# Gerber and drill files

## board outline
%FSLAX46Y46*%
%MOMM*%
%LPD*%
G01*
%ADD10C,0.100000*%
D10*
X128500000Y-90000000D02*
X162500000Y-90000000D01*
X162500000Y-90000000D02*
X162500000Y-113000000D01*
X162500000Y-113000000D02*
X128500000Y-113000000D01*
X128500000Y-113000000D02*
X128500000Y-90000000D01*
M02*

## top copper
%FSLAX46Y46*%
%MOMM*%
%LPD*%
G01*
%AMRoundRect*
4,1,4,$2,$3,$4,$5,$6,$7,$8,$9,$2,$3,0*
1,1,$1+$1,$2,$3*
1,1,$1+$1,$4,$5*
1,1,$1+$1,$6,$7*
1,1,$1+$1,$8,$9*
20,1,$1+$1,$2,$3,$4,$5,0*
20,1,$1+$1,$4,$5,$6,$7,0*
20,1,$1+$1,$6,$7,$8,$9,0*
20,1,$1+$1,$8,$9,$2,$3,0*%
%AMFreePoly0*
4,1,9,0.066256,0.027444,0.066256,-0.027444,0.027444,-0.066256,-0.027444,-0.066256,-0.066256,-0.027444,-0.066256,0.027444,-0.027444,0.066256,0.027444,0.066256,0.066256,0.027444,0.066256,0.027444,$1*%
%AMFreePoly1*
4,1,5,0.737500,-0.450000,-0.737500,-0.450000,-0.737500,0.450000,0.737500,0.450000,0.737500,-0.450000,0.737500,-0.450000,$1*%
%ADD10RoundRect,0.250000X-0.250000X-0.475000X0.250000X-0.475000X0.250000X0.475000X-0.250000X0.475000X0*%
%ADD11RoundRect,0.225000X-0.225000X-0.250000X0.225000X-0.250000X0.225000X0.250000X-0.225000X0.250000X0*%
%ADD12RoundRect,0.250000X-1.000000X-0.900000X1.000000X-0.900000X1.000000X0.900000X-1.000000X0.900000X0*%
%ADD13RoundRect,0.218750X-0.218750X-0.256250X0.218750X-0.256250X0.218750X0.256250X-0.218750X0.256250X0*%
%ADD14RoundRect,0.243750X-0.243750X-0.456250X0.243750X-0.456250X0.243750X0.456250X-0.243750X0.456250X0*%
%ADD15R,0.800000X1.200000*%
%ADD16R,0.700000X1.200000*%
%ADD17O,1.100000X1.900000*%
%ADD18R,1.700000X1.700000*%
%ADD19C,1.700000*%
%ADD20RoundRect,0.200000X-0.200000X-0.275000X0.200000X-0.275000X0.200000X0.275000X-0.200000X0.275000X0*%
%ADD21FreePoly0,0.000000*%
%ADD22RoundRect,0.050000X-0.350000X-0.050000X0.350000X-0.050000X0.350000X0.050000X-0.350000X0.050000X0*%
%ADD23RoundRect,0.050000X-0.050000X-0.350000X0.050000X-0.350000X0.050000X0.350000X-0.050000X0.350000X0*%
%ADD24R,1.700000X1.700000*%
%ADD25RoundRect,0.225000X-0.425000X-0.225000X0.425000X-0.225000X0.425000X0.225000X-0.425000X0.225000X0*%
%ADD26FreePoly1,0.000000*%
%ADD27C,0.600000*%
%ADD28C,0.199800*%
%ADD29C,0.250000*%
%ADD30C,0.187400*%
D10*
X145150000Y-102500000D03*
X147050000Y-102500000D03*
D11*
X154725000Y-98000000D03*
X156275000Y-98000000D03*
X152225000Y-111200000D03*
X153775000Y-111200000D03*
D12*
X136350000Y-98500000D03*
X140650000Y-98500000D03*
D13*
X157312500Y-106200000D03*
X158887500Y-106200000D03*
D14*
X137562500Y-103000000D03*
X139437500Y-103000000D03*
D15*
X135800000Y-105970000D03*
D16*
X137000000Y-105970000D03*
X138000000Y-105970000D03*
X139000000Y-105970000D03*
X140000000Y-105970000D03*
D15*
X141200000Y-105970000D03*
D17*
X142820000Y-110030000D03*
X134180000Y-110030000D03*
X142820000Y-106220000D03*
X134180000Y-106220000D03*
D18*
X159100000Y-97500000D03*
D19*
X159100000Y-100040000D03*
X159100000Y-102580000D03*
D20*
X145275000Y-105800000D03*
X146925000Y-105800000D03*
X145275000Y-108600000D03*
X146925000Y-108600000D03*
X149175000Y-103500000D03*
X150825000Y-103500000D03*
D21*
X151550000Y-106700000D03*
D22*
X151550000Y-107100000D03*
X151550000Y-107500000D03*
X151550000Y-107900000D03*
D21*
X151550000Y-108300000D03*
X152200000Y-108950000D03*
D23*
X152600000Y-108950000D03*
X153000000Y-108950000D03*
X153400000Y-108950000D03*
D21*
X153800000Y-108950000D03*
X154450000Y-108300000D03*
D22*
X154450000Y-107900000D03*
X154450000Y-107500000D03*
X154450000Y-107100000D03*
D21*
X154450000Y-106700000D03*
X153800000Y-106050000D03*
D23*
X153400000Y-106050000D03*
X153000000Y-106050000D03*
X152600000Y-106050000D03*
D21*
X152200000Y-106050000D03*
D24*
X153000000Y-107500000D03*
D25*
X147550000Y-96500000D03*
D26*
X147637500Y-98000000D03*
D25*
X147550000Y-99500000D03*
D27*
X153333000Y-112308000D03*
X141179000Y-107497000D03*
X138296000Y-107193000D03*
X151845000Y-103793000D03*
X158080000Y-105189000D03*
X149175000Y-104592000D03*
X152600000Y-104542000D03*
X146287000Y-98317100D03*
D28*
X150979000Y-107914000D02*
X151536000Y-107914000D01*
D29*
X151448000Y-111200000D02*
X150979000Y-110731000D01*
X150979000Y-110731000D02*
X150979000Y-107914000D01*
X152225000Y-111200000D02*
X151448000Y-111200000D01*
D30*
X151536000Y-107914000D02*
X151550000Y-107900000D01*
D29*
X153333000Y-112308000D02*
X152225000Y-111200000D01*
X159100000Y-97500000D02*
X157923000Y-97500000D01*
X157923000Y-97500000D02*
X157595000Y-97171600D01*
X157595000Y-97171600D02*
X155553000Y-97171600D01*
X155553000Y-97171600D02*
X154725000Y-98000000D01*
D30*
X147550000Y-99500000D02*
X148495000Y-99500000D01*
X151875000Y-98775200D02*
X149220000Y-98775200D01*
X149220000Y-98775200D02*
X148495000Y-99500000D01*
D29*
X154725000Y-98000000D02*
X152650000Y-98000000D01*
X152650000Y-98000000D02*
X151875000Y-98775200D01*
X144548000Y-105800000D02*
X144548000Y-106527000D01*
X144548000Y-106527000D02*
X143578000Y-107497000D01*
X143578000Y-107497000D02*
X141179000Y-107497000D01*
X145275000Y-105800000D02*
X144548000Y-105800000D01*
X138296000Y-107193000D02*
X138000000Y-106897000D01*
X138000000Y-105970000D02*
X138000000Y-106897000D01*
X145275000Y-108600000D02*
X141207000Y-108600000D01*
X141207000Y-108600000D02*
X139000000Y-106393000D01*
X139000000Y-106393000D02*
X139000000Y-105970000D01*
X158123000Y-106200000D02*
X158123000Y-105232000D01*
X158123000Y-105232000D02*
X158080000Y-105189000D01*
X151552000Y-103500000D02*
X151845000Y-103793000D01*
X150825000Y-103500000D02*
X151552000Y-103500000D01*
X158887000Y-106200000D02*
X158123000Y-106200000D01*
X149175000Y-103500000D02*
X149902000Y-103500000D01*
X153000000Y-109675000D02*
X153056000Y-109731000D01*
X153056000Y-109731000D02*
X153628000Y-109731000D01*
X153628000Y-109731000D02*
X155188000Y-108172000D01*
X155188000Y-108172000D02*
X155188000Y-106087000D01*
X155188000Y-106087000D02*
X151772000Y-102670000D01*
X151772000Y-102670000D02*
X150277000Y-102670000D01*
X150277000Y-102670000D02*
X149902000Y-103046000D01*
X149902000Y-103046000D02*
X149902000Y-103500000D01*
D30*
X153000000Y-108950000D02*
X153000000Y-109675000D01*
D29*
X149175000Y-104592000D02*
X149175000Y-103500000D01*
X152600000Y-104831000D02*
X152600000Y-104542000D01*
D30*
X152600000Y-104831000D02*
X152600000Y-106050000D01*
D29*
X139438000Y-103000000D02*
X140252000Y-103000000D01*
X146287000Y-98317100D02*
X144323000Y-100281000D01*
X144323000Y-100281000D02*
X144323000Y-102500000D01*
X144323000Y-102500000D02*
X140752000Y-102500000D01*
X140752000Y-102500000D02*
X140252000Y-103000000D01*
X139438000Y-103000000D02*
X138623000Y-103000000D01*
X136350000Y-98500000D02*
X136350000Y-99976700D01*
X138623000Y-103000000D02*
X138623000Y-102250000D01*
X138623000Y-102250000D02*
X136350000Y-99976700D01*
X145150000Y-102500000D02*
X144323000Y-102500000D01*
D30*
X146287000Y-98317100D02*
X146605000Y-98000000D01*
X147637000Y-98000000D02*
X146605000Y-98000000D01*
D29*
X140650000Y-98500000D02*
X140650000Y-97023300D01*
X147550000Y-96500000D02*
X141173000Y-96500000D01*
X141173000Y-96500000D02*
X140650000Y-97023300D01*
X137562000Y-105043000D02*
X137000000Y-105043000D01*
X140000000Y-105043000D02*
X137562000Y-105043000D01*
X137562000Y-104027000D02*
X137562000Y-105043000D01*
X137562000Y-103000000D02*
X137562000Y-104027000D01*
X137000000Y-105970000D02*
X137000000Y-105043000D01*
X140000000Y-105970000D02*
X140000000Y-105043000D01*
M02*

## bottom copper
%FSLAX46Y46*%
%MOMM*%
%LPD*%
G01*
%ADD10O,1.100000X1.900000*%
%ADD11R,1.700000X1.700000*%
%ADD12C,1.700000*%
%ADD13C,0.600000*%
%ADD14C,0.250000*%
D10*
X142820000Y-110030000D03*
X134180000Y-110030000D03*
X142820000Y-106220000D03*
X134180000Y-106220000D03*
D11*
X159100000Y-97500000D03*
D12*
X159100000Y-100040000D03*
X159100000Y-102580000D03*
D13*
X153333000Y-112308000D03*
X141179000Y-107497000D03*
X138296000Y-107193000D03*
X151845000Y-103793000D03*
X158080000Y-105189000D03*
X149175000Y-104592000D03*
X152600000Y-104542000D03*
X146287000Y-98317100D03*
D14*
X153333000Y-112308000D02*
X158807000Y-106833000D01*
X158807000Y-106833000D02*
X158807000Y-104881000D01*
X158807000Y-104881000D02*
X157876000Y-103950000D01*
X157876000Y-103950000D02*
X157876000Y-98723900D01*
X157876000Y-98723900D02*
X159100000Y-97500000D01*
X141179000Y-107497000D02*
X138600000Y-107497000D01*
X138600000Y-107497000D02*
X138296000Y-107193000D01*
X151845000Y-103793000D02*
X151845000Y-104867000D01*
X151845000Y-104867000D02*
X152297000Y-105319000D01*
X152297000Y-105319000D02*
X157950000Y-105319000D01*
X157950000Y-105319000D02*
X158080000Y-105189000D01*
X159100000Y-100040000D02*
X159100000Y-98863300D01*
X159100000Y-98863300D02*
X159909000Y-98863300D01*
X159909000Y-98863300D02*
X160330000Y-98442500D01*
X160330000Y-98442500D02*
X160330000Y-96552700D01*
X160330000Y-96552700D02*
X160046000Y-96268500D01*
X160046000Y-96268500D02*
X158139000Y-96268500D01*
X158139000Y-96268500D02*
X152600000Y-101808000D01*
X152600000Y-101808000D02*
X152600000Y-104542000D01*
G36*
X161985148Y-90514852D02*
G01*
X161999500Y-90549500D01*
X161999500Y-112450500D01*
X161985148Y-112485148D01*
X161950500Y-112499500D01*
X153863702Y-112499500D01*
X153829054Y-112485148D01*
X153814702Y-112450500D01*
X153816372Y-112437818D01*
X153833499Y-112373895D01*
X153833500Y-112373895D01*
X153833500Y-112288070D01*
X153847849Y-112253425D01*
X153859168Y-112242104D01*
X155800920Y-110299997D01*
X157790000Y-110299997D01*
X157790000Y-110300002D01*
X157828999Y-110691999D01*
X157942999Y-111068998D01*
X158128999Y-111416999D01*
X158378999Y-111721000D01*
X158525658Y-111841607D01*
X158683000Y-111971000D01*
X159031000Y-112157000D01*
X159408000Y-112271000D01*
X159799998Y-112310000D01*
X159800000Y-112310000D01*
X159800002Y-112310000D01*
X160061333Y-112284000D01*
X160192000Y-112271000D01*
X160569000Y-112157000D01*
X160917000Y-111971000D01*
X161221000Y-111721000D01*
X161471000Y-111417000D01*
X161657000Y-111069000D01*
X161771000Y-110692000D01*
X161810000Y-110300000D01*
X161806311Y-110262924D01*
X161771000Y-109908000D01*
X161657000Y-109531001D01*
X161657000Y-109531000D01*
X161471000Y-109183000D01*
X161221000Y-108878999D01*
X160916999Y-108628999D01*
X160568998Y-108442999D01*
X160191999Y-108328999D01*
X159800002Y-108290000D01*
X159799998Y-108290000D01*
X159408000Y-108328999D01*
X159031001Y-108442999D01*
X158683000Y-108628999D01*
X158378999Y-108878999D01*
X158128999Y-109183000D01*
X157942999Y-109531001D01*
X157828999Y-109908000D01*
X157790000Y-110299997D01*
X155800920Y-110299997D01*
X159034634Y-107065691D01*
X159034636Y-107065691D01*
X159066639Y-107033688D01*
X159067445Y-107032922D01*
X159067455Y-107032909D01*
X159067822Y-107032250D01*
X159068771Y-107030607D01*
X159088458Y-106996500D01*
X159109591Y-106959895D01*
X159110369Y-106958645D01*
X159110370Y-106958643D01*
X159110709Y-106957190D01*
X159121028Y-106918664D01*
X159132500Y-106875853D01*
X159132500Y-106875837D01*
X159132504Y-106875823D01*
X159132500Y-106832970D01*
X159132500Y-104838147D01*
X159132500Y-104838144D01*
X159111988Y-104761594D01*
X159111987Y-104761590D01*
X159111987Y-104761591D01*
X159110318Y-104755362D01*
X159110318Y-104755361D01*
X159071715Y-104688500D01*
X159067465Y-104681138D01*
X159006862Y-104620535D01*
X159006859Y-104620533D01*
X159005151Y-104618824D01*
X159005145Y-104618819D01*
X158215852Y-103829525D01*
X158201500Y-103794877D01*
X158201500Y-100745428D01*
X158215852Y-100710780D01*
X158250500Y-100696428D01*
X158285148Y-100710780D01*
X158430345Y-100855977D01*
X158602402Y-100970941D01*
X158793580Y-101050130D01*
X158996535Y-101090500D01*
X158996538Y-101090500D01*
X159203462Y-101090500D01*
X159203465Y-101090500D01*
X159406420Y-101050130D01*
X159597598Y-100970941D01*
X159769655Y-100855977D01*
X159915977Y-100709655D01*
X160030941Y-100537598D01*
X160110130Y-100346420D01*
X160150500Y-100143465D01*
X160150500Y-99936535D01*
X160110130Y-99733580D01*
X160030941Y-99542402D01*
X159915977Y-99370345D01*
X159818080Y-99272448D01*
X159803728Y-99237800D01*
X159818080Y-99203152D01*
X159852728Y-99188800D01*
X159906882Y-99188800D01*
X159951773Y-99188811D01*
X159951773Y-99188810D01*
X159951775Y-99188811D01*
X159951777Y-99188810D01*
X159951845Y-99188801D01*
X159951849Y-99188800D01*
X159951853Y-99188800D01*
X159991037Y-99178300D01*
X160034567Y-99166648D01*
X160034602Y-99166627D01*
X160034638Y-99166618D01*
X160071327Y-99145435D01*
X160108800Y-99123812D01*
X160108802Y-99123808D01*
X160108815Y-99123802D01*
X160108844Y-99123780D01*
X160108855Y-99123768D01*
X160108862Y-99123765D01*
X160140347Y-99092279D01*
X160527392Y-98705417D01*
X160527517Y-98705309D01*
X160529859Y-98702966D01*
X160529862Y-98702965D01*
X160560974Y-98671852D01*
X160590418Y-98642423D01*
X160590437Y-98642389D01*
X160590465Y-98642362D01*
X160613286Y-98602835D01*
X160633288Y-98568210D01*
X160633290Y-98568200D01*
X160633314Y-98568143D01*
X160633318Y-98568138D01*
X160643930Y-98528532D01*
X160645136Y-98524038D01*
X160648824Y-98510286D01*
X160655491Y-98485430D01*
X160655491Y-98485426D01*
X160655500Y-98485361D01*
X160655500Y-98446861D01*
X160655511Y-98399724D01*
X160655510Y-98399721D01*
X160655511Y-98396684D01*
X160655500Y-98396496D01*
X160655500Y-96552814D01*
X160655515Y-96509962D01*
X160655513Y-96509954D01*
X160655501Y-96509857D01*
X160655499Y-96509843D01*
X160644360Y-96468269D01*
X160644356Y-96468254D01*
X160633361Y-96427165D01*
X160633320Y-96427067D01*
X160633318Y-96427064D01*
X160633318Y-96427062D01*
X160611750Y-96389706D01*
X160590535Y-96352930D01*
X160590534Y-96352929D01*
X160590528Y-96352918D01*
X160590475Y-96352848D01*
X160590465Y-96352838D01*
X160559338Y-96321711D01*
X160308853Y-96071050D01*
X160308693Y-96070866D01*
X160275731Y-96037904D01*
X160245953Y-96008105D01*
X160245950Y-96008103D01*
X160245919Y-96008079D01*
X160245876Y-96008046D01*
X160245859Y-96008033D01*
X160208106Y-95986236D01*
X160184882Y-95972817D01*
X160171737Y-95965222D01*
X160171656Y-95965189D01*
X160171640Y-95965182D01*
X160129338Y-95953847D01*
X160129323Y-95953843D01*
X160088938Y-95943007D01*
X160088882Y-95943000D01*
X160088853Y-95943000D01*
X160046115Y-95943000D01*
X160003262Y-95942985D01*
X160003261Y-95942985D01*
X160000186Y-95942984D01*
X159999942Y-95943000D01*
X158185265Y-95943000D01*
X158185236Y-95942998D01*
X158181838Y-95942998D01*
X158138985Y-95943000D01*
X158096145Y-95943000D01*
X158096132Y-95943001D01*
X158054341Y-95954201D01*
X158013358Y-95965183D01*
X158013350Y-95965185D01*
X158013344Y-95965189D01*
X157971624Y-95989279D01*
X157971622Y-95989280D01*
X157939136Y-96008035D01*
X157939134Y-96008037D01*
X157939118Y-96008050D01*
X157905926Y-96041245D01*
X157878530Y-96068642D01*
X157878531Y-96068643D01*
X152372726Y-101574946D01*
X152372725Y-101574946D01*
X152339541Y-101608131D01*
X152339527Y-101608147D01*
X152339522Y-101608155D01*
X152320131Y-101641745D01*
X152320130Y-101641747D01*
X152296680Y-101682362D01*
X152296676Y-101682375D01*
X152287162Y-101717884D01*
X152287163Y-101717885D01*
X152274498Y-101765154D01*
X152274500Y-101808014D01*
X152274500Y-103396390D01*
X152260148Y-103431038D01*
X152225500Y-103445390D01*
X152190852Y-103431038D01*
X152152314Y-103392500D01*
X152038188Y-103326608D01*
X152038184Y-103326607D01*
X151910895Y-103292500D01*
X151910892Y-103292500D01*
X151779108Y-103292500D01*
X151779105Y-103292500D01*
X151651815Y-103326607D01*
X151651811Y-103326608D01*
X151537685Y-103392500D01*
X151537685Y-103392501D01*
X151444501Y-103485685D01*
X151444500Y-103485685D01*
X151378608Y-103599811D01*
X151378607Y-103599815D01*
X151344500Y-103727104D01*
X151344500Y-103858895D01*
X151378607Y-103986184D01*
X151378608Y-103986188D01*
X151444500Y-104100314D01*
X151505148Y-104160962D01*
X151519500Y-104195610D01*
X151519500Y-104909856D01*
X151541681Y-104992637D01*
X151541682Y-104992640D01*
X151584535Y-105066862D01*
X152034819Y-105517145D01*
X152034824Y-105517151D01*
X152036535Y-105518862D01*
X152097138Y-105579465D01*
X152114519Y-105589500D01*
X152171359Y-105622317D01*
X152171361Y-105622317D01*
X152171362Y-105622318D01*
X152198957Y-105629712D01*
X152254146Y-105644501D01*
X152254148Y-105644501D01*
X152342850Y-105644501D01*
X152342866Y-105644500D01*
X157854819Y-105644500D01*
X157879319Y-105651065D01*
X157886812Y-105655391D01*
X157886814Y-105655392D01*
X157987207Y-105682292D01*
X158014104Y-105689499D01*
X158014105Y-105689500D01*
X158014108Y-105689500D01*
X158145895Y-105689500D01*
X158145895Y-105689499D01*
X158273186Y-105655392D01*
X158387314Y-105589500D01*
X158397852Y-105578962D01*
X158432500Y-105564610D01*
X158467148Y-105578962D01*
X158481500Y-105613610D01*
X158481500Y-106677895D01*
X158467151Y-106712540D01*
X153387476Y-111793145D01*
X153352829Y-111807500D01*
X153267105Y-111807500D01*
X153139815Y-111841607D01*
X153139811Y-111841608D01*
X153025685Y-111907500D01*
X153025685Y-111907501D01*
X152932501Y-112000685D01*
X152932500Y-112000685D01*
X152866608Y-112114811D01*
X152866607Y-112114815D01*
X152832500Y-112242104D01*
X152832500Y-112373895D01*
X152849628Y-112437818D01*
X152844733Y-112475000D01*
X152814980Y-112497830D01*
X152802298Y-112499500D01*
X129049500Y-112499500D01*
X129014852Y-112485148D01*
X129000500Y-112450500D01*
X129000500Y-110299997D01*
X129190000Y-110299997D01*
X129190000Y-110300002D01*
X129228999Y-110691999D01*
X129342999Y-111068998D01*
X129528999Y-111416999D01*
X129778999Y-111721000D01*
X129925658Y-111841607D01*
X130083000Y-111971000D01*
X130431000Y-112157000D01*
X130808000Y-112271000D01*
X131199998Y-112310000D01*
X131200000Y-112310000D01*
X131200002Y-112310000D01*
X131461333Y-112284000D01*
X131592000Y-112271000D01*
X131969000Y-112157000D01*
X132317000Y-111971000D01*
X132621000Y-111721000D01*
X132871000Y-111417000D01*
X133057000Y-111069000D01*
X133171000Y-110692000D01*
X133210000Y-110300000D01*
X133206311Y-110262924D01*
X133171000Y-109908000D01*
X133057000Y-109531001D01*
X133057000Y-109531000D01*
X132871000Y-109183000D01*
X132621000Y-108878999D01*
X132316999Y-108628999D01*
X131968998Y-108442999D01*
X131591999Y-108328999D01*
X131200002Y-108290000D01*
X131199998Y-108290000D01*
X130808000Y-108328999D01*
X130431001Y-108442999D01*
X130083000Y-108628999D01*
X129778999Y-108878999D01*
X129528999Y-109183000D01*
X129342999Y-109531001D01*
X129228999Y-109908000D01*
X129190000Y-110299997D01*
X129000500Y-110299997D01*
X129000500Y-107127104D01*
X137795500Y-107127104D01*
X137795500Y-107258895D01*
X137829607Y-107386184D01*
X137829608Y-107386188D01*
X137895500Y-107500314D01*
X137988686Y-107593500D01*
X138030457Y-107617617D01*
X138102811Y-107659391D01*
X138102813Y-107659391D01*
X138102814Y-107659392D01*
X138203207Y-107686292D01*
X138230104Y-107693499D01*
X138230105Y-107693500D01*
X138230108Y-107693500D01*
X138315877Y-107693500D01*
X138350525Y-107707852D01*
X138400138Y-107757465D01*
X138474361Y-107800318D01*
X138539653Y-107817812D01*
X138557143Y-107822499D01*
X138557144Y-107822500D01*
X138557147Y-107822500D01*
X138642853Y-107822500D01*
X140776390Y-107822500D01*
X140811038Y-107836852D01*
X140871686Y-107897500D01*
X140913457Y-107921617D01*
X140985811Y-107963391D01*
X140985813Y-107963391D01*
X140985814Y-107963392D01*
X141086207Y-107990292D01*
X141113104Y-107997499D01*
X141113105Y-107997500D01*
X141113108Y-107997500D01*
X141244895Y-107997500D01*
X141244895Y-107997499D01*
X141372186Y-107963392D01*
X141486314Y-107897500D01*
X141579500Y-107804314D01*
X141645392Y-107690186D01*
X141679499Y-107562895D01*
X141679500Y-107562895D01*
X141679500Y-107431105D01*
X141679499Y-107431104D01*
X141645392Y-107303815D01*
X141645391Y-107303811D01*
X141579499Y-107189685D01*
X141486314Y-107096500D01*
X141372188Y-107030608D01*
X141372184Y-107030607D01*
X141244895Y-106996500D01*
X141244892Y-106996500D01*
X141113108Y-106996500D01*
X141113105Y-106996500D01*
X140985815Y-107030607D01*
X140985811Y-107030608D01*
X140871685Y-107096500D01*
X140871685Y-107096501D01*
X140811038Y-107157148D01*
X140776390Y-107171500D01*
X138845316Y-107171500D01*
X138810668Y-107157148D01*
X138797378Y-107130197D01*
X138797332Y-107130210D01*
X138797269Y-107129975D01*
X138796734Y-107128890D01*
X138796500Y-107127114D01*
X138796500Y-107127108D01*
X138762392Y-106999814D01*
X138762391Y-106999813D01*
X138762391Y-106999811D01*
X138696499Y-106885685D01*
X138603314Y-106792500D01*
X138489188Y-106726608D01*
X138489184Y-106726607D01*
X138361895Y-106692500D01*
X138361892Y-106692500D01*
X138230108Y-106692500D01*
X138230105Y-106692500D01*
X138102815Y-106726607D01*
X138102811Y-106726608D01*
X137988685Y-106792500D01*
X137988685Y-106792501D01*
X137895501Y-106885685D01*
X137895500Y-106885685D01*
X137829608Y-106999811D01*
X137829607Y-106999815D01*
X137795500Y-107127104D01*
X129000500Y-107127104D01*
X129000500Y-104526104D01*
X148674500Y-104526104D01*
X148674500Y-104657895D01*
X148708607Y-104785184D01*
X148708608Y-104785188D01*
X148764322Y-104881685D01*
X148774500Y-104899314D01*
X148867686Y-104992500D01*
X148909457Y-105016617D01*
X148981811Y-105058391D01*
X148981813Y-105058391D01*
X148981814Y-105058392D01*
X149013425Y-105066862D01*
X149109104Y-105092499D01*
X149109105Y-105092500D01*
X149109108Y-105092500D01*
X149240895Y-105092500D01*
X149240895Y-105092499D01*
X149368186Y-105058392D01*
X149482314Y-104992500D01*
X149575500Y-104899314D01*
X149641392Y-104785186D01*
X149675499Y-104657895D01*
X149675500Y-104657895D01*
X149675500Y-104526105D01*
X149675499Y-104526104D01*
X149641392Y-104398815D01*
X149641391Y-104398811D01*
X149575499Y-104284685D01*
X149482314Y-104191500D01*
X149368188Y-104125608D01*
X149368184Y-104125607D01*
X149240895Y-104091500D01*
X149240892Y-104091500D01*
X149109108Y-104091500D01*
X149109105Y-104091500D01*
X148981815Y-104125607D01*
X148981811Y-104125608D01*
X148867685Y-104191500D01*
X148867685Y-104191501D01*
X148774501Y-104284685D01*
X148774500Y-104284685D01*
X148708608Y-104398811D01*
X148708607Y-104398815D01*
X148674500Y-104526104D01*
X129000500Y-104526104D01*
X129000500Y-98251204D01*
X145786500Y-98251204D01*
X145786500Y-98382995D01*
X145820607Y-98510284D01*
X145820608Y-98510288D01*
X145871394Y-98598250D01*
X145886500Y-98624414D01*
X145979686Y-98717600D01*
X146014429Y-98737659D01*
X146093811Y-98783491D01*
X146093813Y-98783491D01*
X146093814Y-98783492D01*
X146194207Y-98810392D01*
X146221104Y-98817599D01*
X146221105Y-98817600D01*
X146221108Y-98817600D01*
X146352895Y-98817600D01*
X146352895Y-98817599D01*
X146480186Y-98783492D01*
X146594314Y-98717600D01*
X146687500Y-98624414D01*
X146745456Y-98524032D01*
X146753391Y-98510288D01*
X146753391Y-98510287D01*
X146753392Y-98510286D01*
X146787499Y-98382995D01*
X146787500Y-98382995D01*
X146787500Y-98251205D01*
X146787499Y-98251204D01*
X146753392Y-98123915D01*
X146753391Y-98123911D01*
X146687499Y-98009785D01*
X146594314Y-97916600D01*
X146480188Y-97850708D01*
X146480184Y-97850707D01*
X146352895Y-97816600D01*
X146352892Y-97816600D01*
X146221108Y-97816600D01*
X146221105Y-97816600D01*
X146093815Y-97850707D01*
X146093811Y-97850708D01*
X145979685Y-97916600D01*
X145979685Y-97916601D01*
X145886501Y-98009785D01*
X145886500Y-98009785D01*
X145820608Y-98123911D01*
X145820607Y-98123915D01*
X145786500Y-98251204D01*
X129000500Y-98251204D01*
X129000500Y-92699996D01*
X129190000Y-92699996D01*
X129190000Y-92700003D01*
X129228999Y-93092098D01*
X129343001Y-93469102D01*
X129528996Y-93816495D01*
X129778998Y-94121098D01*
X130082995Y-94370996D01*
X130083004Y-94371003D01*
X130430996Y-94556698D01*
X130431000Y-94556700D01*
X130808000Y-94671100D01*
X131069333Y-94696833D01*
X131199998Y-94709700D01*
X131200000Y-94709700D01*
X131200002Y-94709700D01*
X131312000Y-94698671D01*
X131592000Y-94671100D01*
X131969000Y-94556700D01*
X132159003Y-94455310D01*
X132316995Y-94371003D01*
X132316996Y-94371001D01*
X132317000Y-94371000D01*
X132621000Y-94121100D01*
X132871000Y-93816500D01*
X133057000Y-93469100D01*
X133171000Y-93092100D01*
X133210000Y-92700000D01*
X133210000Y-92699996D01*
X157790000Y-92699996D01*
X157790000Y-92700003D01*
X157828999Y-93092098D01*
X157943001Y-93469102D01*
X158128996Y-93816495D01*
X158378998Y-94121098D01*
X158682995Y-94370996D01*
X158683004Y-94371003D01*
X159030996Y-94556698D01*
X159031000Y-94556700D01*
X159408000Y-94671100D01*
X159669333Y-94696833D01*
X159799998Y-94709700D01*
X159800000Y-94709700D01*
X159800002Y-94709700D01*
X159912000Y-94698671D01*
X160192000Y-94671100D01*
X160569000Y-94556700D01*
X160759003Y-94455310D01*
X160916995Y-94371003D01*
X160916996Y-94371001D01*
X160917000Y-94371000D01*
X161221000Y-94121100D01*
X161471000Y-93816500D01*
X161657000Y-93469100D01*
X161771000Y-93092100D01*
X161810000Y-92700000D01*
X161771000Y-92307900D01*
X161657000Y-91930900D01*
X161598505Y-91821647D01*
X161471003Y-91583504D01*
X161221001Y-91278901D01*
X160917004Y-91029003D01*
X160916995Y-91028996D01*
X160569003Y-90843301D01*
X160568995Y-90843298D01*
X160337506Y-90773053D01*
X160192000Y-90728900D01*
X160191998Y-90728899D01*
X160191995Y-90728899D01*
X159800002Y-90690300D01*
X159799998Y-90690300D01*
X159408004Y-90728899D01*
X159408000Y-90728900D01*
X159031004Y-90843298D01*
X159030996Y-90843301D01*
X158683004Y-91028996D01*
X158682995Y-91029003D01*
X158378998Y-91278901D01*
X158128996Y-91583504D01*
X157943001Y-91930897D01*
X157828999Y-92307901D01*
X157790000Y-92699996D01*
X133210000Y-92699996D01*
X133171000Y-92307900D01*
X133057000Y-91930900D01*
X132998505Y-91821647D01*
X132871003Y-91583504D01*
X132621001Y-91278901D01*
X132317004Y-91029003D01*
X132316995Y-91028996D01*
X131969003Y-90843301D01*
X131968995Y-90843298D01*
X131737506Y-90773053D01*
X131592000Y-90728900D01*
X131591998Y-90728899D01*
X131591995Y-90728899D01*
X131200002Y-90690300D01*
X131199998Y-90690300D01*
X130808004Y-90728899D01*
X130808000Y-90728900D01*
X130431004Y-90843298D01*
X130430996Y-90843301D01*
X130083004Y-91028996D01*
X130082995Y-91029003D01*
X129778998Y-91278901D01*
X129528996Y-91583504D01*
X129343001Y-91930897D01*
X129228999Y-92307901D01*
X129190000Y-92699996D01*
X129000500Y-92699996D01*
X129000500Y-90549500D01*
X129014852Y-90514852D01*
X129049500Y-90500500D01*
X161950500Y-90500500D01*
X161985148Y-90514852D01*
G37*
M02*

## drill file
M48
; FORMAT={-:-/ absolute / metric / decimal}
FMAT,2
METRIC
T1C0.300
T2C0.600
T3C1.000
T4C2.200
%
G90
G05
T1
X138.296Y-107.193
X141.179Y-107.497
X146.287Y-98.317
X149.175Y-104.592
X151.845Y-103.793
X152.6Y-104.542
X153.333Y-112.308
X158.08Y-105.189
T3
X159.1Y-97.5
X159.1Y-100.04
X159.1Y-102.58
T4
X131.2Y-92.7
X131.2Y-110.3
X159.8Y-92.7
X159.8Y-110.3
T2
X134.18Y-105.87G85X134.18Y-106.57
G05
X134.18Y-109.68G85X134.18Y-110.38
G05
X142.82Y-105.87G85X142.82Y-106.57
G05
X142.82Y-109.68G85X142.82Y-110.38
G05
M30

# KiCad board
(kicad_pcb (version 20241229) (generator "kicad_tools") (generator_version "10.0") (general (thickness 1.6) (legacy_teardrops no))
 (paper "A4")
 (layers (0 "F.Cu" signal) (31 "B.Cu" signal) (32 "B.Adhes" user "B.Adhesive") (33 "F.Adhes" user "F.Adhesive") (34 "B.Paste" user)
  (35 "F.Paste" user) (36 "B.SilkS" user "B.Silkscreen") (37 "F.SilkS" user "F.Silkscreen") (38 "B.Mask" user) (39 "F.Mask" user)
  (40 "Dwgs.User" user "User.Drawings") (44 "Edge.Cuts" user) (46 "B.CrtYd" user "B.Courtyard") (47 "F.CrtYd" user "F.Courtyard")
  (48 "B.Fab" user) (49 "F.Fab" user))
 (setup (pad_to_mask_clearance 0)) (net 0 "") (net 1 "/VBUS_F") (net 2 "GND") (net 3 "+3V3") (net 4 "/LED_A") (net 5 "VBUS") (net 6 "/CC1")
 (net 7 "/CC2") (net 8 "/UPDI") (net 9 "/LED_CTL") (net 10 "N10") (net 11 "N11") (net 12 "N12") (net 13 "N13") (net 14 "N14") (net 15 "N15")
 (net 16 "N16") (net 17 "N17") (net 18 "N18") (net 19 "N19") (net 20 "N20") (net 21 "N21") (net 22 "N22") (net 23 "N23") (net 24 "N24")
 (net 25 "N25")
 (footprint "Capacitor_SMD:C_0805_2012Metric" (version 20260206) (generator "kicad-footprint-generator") (layer "F.Cu") (at 146.1 102.5)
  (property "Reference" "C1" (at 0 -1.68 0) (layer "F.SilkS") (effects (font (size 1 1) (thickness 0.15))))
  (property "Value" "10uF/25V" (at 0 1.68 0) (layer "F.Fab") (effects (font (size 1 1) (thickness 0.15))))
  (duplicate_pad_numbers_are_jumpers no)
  (pad "1" smd roundrect (at -0.95 0) (size 1 1.45) (layers "F.Cu" "F.Mask" "F.Paste") (roundrect_rratio 0.25) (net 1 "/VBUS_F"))
  (pad "2" smd roundrect (at 0.95 0) (size 1 1.45) (layers "F.Cu" "F.Mask" "F.Paste") (roundrect_rratio 0.25) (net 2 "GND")))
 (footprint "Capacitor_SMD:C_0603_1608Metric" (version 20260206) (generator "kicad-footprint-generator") (layer "F.Cu") (at 155.5 98)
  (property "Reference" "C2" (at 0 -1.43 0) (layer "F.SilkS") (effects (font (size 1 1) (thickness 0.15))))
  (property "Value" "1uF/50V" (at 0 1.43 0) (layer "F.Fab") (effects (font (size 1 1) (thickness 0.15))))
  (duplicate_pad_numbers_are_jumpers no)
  (pad "1" smd roundrect (at -0.775 0) (size 0.9 0.95) (layers "F.Cu" "F.Mask" "F.Paste") (roundrect_rratio 0.25) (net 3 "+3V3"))
  (pad "2" smd roundrect (at 0.775 0) (size 0.9 0.95) (layers "F.Cu" "F.Mask" "F.Paste") (roundrect_rratio 0.25) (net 2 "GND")))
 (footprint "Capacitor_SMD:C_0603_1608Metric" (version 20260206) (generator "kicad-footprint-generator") (layer "F.Cu") (at 153 111.2)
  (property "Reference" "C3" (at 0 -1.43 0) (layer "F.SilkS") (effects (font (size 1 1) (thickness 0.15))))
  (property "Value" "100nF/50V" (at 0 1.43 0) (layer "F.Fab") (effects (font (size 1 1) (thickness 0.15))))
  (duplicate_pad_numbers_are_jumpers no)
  (pad "1" smd roundrect (at -0.775 0) (size 0.9 0.95) (layers "F.Cu" "F.Mask" "F.Paste") (roundrect_rratio 0.25) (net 3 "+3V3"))
  (pad "2" smd roundrect (at 0.775 0) (size 0.9 0.95) (layers "F.Cu" "F.Mask" "F.Paste") (roundrect_rratio 0.25) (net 2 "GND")))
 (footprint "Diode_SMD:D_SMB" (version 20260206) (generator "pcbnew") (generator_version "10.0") (layer "F.Cu") (at 138.5 98.5)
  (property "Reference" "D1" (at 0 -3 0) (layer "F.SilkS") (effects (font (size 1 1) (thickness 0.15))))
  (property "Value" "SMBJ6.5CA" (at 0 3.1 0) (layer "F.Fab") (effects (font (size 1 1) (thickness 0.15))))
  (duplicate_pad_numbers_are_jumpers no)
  (pad "1" smd roundrect (at -2.15 0) (size 2.5 2.3) (layers "F.Cu" "F.Mask" "F.Paste") (roundrect_rratio 0.1086956522) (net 1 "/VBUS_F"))
  (pad "2" smd roundrect (at 2.15 0) (size 2.5 2.3) (layers "F.Cu" "F.Mask" "F.Paste") (roundrect_rratio 0.1086956522) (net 2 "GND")))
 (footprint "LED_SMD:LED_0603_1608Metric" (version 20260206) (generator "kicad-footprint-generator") (layer "F.Cu") (at 158.1 106.2)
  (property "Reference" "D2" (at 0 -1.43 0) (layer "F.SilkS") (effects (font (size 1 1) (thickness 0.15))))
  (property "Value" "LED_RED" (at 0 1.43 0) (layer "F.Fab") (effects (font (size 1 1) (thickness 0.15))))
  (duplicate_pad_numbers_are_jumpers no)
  (pad "1" smd roundrect (at -0.7875 0) (size 0.875 0.95) (layers "F.Cu" "F.Mask" "F.Paste") (roundrect_rratio 0.25) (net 2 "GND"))
  (pad "2" smd roundrect (at 0.7875 0) (size 0.875 0.95) (layers "F.Cu" "F.Mask" "F.Paste") (roundrect_rratio 0.25) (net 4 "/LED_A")))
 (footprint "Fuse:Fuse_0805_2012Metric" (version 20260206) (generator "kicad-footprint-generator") (layer "F.Cu") (at 138.5 103)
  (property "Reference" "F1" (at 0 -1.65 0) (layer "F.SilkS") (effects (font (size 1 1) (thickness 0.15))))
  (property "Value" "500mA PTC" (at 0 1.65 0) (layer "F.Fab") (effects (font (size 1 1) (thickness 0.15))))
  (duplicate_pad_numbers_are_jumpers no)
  (pad "1" smd roundrect (at -0.9375 0) (size 0.975 1.4) (layers "F.Cu" "F.Mask" "F.Paste") (roundrect_rratio 0.25) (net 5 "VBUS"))
  (pad "2" smd roundrect (at 0.9375 0) (size 0.975 1.4) (layers "F.Cu" "F.Mask" "F.Paste") (roundrect_rratio 0.25) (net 1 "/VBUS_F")))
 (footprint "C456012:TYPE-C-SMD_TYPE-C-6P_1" (layer "F.Cu") (at 138.5 108)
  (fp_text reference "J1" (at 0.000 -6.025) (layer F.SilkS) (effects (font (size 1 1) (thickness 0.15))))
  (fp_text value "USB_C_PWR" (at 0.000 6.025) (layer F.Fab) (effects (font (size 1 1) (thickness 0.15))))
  (pad B12 smd rect (at -2.70 -2.03 0.00) (size 0.800 1.200) (layers F.Cu F.Paste F.Mask) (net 2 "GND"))
  (pad B9 smd rect (at -1.50 -2.03 0.00) (size 0.700 1.200) (layers F.Cu F.Paste F.Mask) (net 5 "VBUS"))
  (pad A5 smd rect (at -0.50 -2.03 0.00) (size 0.700 1.200) (layers F.Cu F.Paste F.Mask) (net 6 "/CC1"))
  (pad B5 smd rect (at 0.50 -2.03 0.00) (size 0.700 1.200) (layers F.Cu F.Paste F.Mask) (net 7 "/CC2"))
  (pad A9 smd rect (at 1.50 -2.03 0.00) (size 0.700 1.200) (layers F.Cu F.Paste F.Mask) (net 5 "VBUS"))
  (pad A12 smd rect (at 2.70 -2.03 0.00) (size 0.800 1.200) (layers F.Cu F.Paste F.Mask) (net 2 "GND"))
  (pad 7 thru_hole oval (at 4.32 2.03 0.00) (size 1.100 1.900) (layers *.Cu *.Mask) (drill oval 0.599998 1.299997) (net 2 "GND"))
  (pad 7 thru_hole oval (at -4.32 2.03 0.00) (size 1.100 1.900) (layers *.Cu *.Mask) (drill oval 0.599998 1.299997) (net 2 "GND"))
  (pad 7 thru_hole oval (at 4.32 -1.78 0.00) (size 1.100 1.900) (layers *.Cu *.Mask) (drill oval 0.599998 1.299997) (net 2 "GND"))
  (pad 7 thru_hole oval (at -4.32 -1.78 0.00) (size 1.100 1.900) (layers *.Cu *.Mask) (drill oval 0.599998 1.299997) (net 2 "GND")))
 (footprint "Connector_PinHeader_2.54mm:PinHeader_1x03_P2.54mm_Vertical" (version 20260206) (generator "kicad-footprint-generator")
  (layer "F.Cu") (at 159.1 97.5)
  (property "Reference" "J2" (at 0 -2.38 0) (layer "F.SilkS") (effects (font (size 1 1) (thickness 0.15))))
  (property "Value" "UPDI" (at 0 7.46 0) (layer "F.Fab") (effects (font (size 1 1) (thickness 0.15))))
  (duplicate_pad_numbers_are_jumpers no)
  (pad "1" thru_hole rect (at 0 0) (size 1.7 1.7) (drill 1) (layers "*.Cu" "*.Mask") (remove_unused_layers no) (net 3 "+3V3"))
  (pad "2" thru_hole circle (at 0 2.54) (size 1.7 1.7) (drill 1) (layers "*.Cu" "*.Mask") (remove_unused_layers no) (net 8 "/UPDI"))
  (pad "3" thru_hole circle (at 0 5.08) (size 1.7 1.7) (drill 1) (layers "*.Cu" "*.Mask") (remove_unused_layers no) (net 2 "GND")))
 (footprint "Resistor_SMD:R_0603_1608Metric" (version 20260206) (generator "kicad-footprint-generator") (layer "F.Cu") (at 146.1 105.8)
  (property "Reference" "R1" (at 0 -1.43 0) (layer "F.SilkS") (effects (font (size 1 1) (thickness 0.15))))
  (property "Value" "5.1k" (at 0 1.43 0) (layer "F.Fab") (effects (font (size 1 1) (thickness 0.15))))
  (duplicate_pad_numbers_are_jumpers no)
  (pad "1" smd roundrect (at -0.825 0) (size 0.8 0.95) (layers "F.Cu" "F.Mask" "F.Paste") (roundrect_rratio 0.25) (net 6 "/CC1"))
  (pad "2" smd roundrect (at 0.825 0) (size 0.8 0.95) (layers "F.Cu" "F.Mask" "F.Paste") (roundrect_rratio 0.25) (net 2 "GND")))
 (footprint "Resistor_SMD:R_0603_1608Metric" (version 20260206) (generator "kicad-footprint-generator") (layer "F.Cu") (at 146.1 108.6)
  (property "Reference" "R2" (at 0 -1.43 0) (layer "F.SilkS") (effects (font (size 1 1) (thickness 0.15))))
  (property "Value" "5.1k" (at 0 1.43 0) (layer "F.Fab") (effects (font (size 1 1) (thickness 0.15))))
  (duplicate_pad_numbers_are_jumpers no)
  (pad "1" smd roundrect (at -0.825 0) (size 0.8 0.95) (layers "F.Cu" "F.Mask" "F.Paste") (roundrect_rratio 0.25) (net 7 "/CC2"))
  (pad "2" smd roundrect (at 0.825 0) (size 0.8 0.95) (layers "F.Cu" "F.Mask" "F.Paste") (roundrect_rratio 0.25) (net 2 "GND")))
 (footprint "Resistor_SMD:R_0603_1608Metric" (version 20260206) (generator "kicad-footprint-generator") (layer "F.Cu") (at 150 103.5)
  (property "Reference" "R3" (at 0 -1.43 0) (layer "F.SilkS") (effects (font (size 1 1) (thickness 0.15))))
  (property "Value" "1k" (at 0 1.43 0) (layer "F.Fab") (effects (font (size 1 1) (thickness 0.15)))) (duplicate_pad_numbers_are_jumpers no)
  (pad "1" smd roundrect (at -0.825 0) (size 0.8 0.95) (layers "F.Cu" "F.Mask" "F.Paste") (roundrect_rratio 0.25) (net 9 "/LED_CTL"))
  (pad "2" smd roundrect (at 0.825 0) (size 0.8 0.95) (layers "F.Cu" "F.Mask" "F.Paste") (roundrect_rratio 0.25) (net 4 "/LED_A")))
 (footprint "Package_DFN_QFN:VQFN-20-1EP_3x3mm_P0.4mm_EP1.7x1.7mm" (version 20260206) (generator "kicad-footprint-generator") (layer "F.Cu")
  (at 153 107.5)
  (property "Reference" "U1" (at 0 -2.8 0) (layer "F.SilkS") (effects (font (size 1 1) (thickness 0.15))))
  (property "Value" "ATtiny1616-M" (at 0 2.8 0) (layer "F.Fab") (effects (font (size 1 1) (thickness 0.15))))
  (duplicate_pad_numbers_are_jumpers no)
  (pad "" smd roundrect (at -0.425 -0.425) (size 0.69 0.69) (layers "F.Paste") (roundrect_rratio 0.25))
  (pad "" smd roundrect (at -0.425 0.425) (size 0.69 0.69) (layers "F.Paste") (roundrect_rratio 0.25))
  (pad "" smd roundrect (at 0.425 -0.425) (size 0.69 0.69) (layers "F.Paste") (roundrect_rratio 0.25))
  (pad "" smd roundrect (at 0.425 0.425) (size 0.69 0.69) (layers "F.Paste") (roundrect_rratio 0.25))
  (pad "1" smd custom (at -1.45 -0.8) (size 0.143431 0.143431) (layers "F.Cu" "F.Mask" "F.Paste")
   (options (clearance outline) (anchor circle)) (primitives) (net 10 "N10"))
  (pad "2" smd roundrect (at -1.45 -0.4) (size 0.8 0.2) (layers "F.Cu" "F.Mask" "F.Paste") (roundrect_rratio 0.25) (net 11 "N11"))
  (pad "3" smd roundrect (at -1.45 0) (size 0.8 0.2) (layers "F.Cu" "F.Mask" "F.Paste") (roundrect_rratio 0.25) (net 2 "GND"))
  (pad "4" smd roundrect (at -1.45 0.4) (size 0.8 0.2) (layers "F.Cu" "F.Mask" "F.Paste") (roundrect_rratio 0.25) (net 3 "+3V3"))
  (pad "5" smd custom (at -1.45 0.8) (size 0.143431 0.143431) (layers "F.Cu" "F.Mask" "F.Paste")
   (options (clearance outline) (anchor circle)) (primitives) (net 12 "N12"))
  (pad "6" smd custom (at -0.8 1.45) (size 0.143431 0.143431) (layers "F.Cu" "F.Mask" "F.Paste")
   (options (clearance outline) (anchor circle)) (primitives) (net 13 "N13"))
  (pad "7" smd roundrect (at -0.4 1.45) (size 0.2 0.8) (layers "F.Cu" "F.Mask" "F.Paste") (roundrect_rratio 0.25) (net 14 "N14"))
  (pad "8" smd roundrect (at 0 1.45) (size 0.2 0.8) (layers "F.Cu" "F.Mask" "F.Paste") (roundrect_rratio 0.25) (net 9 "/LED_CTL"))
  (pad "9" smd roundrect (at 0.4 1.45) (size 0.2 0.8) (layers "F.Cu" "F.Mask" "F.Paste") (roundrect_rratio 0.25) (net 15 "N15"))
  (pad "10" smd custom (at 0.8 1.45) (size 0.143431 0.143431) (layers "F.Cu" "F.Mask" "F.Paste")
   (options (clearance outline) (anchor circle)) (primitives) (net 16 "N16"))
  (pad "11" smd custom (at 1.45 0.8) (size 0.143431 0.143431) (layers "F.Cu" "F.Mask" "F.Paste")
   (options (clearance outline) (anchor circle)) (primitives) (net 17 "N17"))
  (pad "12" smd roundrect (at 1.45 0.4) (size 0.8 0.2) (layers "F.Cu" "F.Mask" "F.Paste") (roundrect_rratio 0.25) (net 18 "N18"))
  (pad "13" smd roundrect (at 1.45 0) (size 0.8 0.2) (layers "F.Cu" "F.Mask" "F.Paste") (roundrect_rratio 0.25) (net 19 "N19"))
  (pad "14" smd roundrect (at 1.45 -0.4) (size 0.8 0.2) (layers "F.Cu" "F.Mask" "F.Paste") (roundrect_rratio 0.25) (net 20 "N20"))
  (pad "15" smd custom (at 1.45 -0.8) (size 0.143431 0.143431) (layers "F.Cu" "F.Mask" "F.Paste")
   (options (clearance outline) (anchor circle)) (primitives) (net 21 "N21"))
  (pad "16" smd custom (at 0.8 -1.45) (size 0.143431 0.143431) (layers "F.Cu" "F.Mask" "F.Paste")
   (options (clearance outline) (anchor circle)) (primitives) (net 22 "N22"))
  (pad "17" smd roundrect (at 0.4 -1.45) (size 0.2 0.8) (layers "F.Cu" "F.Mask" "F.Paste") (roundrect_rratio 0.25) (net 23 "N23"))
  (pad "18" smd roundrect (at 0 -1.45) (size 0.2 0.8) (layers "F.Cu" "F.Mask" "F.Paste") (roundrect_rratio 0.25) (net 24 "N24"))
  (pad "19" smd roundrect (at -0.4 -1.45) (size 0.2 0.8) (layers "F.Cu" "F.Mask" "F.Paste") (roundrect_rratio 0.25) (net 8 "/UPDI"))
  (pad "20" smd custom (at -0.8 -1.45) (size 0.143431 0.143431) (layers "F.Cu" "F.Mask" "F.Paste")
   (options (clearance outline) (anchor circle)) (primitives) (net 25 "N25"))
  (pad "21" smd rect (at 0 0) (size 1.7 1.7) (layers "F.Cu" "F.Mask") (zone_connect 2) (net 2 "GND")))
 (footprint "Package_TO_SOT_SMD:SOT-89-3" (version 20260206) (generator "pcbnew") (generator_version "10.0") (layer "F.Cu") (at 149.5 98)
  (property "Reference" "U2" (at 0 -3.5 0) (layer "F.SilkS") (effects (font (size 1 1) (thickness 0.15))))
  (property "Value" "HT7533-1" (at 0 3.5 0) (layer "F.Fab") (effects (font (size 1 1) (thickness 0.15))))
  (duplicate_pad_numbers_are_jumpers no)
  (pad "1" smd roundrect (at -1.95 -1.5) (size 1.3 0.9) (layers "F.Cu" "F.Mask" "F.Paste") (roundrect_rratio 0.25) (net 2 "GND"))
  (pad "2" smd custom (at -1.8625 0) (size 1.475 0.9) (layers "F.Cu" "F.Mask" "F.Paste") (zone_connect 2) (thermal_bridge_angle 45)
   (options (clearance outline) (anchor rect)) (primitives) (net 1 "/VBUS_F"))
  (pad "3" smd roundrect (at -1.95 1.5) (size 1.3 0.9) (layers "F.Cu" "F.Mask" "F.Paste") (roundrect_rratio 0.25) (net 3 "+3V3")))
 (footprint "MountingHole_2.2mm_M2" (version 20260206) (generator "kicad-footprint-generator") (layer "F.Cu") (at 131.2 92.7)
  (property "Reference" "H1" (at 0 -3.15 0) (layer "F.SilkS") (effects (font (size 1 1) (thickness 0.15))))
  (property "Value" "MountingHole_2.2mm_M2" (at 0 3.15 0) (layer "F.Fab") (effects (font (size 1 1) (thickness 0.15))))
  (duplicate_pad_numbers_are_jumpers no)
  (pad "" np_thru_hole circle (at 0 0) (size 2.2 2.2) (drill 2.2) (layers "*.Cu" "*.Mask")))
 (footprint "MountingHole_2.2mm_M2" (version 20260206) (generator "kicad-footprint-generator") (layer "F.Cu") (at 159.8 92.7)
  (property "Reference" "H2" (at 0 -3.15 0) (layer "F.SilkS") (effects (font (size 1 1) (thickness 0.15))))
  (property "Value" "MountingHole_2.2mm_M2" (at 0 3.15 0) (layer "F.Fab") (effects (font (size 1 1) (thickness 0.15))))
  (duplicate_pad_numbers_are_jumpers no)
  (pad "" np_thru_hole circle (at 0 0) (size 2.2 2.2) (drill 2.2) (layers "*.Cu" "*.Mask")))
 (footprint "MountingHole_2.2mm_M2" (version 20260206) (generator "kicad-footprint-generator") (layer "F.Cu") (at 131.2 110.3)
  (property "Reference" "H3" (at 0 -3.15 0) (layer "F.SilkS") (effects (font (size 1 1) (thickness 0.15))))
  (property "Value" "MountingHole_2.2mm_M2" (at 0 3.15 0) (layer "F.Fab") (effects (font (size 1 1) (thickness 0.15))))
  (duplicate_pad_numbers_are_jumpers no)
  (pad "" np_thru_hole circle (at 0 0) (size 2.2 2.2) (drill 2.2) (layers "*.Cu" "*.Mask")))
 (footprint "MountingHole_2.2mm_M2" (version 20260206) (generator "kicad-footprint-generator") (layer "F.Cu") (at 159.8 110.3)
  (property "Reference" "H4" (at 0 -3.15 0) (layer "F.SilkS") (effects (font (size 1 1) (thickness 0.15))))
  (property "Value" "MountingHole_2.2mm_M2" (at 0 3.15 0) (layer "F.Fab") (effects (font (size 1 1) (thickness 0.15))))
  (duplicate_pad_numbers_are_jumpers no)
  (pad "" np_thru_hole circle (at 0 0) (size 2.2 2.2) (drill 2.2) (layers "*.Cu" "*.Mask")))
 (gr_line (start 128.5 90) (end 162.5 90) (stroke (width 0.1) (type default)) (layer "Edge.Cuts"))
 (gr_line (start 162.5 90) (end 162.5 113) (stroke (width 0.1) (type default)) (layer "Edge.Cuts"))
 (gr_line (start 162.5 113) (end 128.5 113) (stroke (width 0.1) (type default)) (layer "Edge.Cuts"))
 (gr_line (start 128.5 113) (end 128.5 90) (stroke (width 0.1) (type default)) (layer "Edge.Cuts"))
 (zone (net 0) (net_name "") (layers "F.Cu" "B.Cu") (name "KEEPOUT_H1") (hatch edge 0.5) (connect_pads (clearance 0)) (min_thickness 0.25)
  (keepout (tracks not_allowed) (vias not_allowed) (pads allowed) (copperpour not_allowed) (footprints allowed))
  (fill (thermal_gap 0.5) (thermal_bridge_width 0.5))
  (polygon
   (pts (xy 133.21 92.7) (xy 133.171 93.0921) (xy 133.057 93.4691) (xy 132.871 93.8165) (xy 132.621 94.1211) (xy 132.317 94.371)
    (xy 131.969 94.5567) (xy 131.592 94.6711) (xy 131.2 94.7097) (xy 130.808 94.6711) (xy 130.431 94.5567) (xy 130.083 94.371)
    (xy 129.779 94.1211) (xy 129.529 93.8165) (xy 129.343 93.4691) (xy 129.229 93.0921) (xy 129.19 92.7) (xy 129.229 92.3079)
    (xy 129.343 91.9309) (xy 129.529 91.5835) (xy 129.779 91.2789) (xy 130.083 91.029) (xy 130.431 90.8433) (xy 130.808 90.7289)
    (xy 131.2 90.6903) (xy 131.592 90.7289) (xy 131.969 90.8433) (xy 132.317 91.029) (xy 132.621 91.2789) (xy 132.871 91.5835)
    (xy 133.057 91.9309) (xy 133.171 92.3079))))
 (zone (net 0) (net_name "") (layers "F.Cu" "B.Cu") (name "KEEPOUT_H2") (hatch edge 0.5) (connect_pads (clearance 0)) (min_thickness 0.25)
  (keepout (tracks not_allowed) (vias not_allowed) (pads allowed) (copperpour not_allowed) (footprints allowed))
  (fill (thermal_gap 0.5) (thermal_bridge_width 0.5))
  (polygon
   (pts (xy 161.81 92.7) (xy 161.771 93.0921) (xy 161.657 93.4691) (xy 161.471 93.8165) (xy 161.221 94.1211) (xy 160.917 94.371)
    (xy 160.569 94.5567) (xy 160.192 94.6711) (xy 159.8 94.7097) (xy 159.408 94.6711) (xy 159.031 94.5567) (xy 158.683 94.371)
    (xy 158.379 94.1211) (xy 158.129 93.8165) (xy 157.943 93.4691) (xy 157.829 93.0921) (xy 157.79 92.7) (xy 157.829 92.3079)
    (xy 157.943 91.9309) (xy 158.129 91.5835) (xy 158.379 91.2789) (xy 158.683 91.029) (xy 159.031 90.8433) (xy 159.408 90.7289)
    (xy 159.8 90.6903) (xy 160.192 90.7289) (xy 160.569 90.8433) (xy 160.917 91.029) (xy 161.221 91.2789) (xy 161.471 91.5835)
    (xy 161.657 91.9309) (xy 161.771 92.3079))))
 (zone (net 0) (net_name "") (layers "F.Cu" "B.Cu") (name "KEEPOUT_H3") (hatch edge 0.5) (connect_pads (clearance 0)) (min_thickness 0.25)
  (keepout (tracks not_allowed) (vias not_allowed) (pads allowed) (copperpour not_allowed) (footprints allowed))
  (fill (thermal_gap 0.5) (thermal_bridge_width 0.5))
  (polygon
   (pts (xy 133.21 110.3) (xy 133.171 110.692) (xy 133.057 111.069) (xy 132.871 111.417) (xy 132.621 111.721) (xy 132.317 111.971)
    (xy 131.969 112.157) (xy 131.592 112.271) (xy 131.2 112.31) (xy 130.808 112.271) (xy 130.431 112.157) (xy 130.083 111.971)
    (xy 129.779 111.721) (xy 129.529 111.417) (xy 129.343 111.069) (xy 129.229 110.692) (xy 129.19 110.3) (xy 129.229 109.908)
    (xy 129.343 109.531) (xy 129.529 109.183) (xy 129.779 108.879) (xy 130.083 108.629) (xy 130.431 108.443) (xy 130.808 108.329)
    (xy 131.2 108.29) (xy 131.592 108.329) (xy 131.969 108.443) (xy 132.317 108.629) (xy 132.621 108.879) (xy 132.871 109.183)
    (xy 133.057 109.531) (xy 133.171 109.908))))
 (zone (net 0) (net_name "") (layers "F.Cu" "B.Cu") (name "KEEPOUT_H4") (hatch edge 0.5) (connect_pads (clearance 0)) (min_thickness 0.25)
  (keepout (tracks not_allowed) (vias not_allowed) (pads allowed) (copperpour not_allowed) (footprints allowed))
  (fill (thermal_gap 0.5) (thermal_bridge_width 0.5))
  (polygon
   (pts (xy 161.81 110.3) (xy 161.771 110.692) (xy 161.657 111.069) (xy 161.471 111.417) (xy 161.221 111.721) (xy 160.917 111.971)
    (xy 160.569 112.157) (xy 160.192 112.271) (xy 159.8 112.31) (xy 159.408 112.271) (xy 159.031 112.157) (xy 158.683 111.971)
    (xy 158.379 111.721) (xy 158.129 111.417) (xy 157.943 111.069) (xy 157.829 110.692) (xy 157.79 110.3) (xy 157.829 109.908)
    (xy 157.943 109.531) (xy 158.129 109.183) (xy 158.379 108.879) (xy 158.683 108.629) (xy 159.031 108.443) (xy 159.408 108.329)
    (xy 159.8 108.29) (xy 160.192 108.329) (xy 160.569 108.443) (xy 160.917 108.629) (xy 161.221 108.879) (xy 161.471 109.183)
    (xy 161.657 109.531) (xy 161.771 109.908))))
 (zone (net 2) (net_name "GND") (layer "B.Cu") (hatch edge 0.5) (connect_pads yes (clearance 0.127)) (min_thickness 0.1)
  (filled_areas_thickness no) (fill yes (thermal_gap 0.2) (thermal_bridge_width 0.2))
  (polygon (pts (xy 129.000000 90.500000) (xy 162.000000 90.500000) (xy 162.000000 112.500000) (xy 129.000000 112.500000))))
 (segment (start 153.333 112.308) (end 158.807 106.833) (width 0.25) (layer "B.Cu") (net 3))
 (segment (start 158.807 106.833) (end 158.807 104.881) (width 0.25) (layer "B.Cu") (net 3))
 (segment (start 158.807 104.881) (end 157.876 103.95) (width 0.25) (layer "B.Cu") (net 3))
 (segment (start 157.876 103.95) (end 157.876 98.7239) (width 0.25) (layer "B.Cu") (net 3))
 (segment (start 157.876 98.7239) (end 159.1 97.5) (width 0.25) (layer "B.Cu") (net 3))
 (segment (start 150.979 107.914) (end 151.536 107.914) (width 0.1998) (layer "F.Cu") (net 3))
 (segment (start 151.448 111.2) (end 150.979 110.731) (width 0.25) (layer "F.Cu") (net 3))
 (segment (start 150.979 110.731) (end 150.979 107.914) (width 0.25) (layer "F.Cu") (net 3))
 (segment (start 152.225 111.2) (end 151.448 111.2) (width 0.25) (layer "F.Cu") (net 3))
 (segment (start 151.536 107.914) (end 151.55 107.9) (width 0.1874) (layer "F.Cu") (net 3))
 (segment (start 153.333 112.308) (end 152.225 111.2) (width 0.25) (layer "F.Cu") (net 3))
 (segment (start 159.1 97.5) (end 157.923 97.5) (width 0.25) (layer "F.Cu") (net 3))
 (segment (start 157.923 97.5) (end 157.595 97.1716) (width 0.25) (layer "F.Cu") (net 3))
 (segment (start 157.595 97.1716) (end 155.553 97.1716) (width 0.25) (layer "F.Cu") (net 3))
 (segment (start 155.553 97.1716) (end 154.725 98) (width 0.25) (layer "F.Cu") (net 3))
 (segment (start 147.55 99.5) (end 148.495 99.5) (width 0.1874) (layer "F.Cu") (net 3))
 (segment (start 151.875 98.7752) (end 149.22 98.7752) (width 0.1874) (layer "F.Cu") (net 3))
 (segment (start 149.22 98.7752) (end 148.495 99.5) (width 0.1874) (layer "F.Cu") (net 3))
 (segment (start 154.725 98) (end 152.65 98) (width 0.25) (layer "F.Cu") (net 3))
 (segment (start 152.65 98) (end 151.875 98.7752) (width 0.25) (layer "F.Cu") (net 3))
 (segment (start 144.548 105.8) (end 144.548 106.527) (width 0.25) (layer "F.Cu") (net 6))
 (segment (start 144.548 106.527) (end 143.578 107.497) (width 0.25) (layer "F.Cu") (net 6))
 (segment (start 143.578 107.497) (end 141.179 107.497) (width 0.25) (layer "F.Cu") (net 6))
 (segment (start 141.179 107.497) (end 138.6 107.497) (width 0.25) (layer "B.Cu") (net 6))
 (segment (start 138.6 107.497) (end 138.296 107.193) (width 0.25) (layer "B.Cu") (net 6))
 (segment (start 145.275 105.8) (end 144.548 105.8) (width 0.25) (layer "F.Cu") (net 6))
 (segment (start 138.296 107.193) (end 138 106.897) (width 0.25) (layer "F.Cu") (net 6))
 (segment (start 138 105.97) (end 138 106.897) (width 0.25) (layer "F.Cu") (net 6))
 (segment (start 145.275 108.6) (end 141.207 108.6) (width 0.25) (layer "F.Cu") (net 7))
 (segment (start 141.207 108.6) (end 139 106.393) (width 0.25) (layer "F.Cu") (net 7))
 (segment (start 139 106.393) (end 139 105.97) (width 0.25) (layer "F.Cu") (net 7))
 (segment (start 158.123 106.2) (end 158.123 105.232) (width 0.25) (layer "F.Cu") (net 4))
 (segment (start 158.123 105.232) (end 158.08 105.189) (width 0.25) (layer "F.Cu") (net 4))
 (segment (start 151.845 103.793) (end 151.845 104.867) (width 0.25) (layer "B.Cu") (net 4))
 (segment (start 151.845 104.867) (end 152.297 105.319) (width 0.25) (layer "B.Cu") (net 4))
 (segment (start 152.297 105.319) (end 157.95 105.319) (width 0.25) (layer "B.Cu") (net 4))
 (segment (start 157.95 105.319) (end 158.08 105.189) (width 0.25) (layer "B.Cu") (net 4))
 (segment (start 151.552 103.5) (end 151.845 103.793) (width 0.25) (layer "F.Cu") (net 4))
 (segment (start 150.825 103.5) (end 151.552 103.5) (width 0.25) (layer "F.Cu") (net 4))
 (segment (start 158.887 106.2) (end 158.123 106.2) (width 0.25) (layer "F.Cu") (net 4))
 (segment (start 149.175 103.5) (end 149.902 103.5) (width 0.25) (layer "F.Cu") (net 9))
 (segment (start 153 109.675) (end 153.056 109.731) (width 0.25) (layer "F.Cu") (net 9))
 (segment (start 153.056 109.731) (end 153.628 109.731) (width 0.25) (layer "F.Cu") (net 9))
 (segment (start 153.628 109.731) (end 155.188 108.172) (width 0.25) (layer "F.Cu") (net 9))
 (segment (start 155.188 108.172) (end 155.188 106.087) (width 0.25) (layer "F.Cu") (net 9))
 (segment (start 155.188 106.087) (end 151.772 102.67) (width 0.25) (layer "F.Cu") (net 9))
 (segment (start 151.772 102.67) (end 150.277 102.67) (width 0.25) (layer "F.Cu") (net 9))
 (segment (start 150.277 102.67) (end 149.902 103.046) (width 0.25) (layer "F.Cu") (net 9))
 (segment (start 149.902 103.046) (end 149.902 103.5) (width 0.25) (layer "F.Cu") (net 9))
 (segment (start 153 108.95) (end 153 109.675) (width 0.1874) (layer "F.Cu") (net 9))
 (segment (start 149.175 104.592) (end 149.175 103.5) (width 0.25) (layer "F.Cu") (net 9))
 (segment (start 159.1 100.04) (end 159.1 98.8633) (width 0.25) (layer "B.Cu") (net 8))
 (segment (start 152.6 104.831) (end 152.6 104.542) (width 0.25) (layer "F.Cu") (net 8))
 (segment (start 159.1 98.8633) (end 159.909 98.8633) (width 0.25) (layer "B.Cu") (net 8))
 (segment (start 159.909 98.8633) (end 160.33 98.4425) (width 0.25) (layer "B.Cu") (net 8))
 (segment (start 160.33 98.4425) (end 160.33 96.5527) (width 0.25) (layer "B.Cu") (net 8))
 (segment (start 160.33 96.5527) (end 160.046 96.2685) (width 0.25) (layer "B.Cu") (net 8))
 (segment (start 160.046 96.2685) (end 158.139 96.2685) (width 0.25) (layer "B.Cu") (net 8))
 (segment (start 158.139 96.2685) (end 152.6 101.808) (width 0.25) (layer "B.Cu") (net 8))
 (segment (start 152.6 101.808) (end 152.6 104.542) (width 0.25) (layer "B.Cu") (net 8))
 (segment (start 152.6 104.831) (end 152.6 106.05) (width 0.1874) (layer "F.Cu") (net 8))
 (segment (start 139.438 103) (end 140.252 103) (width 0.25) (layer "F.Cu") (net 1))
 (segment (start 146.287 98.3171) (end 144.323 100.281) (width 0.25) (layer "F.Cu") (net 1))
 (segment (start 144.323 100.281) (end 144.323 102.5) (width 0.25) (layer "F.Cu") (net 1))
 (segment (start 144.323 102.5) (end 140.752 102.5) (width 0.25) (layer "F.Cu") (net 1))
 (segment (start 140.752 102.5) (end 140.252 103) (width 0.25) (layer "F.Cu") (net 1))
 (segment (start 139.438 103) (end 138.623 103) (width 0.25) (layer "F.Cu") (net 1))
 (segment (start 136.35 98.5) (end 136.35 99.9767) (width 0.25) (layer "F.Cu") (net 1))
 (segment (start 138.623 103) (end 138.623 102.25) (width 0.25) (layer "F.Cu") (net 1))
 (segment (start 138.623 102.25) (end 136.35 99.9767) (width 0.25) (layer "F.Cu") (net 1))
 (segment (start 145.15 102.5) (end 144.323 102.5) (width 0.25) (layer "F.Cu") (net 1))
 (segment (start 146.287 98.3171) (end 146.605 98) (width 0.1874) (layer "F.Cu") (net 1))
 (segment (start 147.637 98) (end 146.605 98) (width 0.1874) (layer "F.Cu") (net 1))
 (segment (start 140.65 98.5) (end 140.65 97.0233) (width 0.25) (layer "F.Cu") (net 2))
 (segment (start 147.55 96.5) (end 141.173 96.5) (width 0.25) (layer "F.Cu") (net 2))
 (segment (start 141.173 96.5) (end 140.65 97.0233) (width 0.25) (layer "F.Cu") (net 2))
 (segment (start 137.562 105.043) (end 137 105.043) (width 0.25) (layer "F.Cu") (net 5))
 (segment (start 140 105.043) (end 137.562 105.043) (width 0.25) (layer "F.Cu") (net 5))
 (segment (start 137.562 104.027) (end 137.562 105.043) (width 0.25) (layer "F.Cu") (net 5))
 (segment (start 137.562 103) (end 137.562 104.027) (width 0.25) (layer "F.Cu") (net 5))
 (segment (start 137 105.97) (end 137 105.043) (width 0.25) (layer "F.Cu") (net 5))
 (segment (start 140 105.97) (end 140 105.043) (width 0.25) (layer "F.Cu") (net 5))
 (via (at 153.333 112.308) (size 0.6) (drill 0.3) (layers "F.Cu" "B.Cu") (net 3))
 (via (at 141.179 107.497) (size 0.6) (drill 0.3) (layers "F.Cu" "B.Cu") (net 6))
 (via (at 138.296 107.193) (size 0.6) (drill 0.3) (layers "F.Cu" "B.Cu") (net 6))
 (via (at 151.845 103.793) (size 0.6) (drill 0.3) (layers "F.Cu" "B.Cu") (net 4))
 (via (at 158.08 105.189) (size 0.6) (drill 0.3) (layers "F.Cu" "B.Cu") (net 4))
 (via (at 149.175 104.592) (size 0.6) (drill 0.3) (layers "F.Cu" "B.Cu") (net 9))
 (via (at 152.6 104.542) (size 0.6) (drill 0.3) (layers "F.Cu" "B.Cu") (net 8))
 (via (at 146.287 98.3171) (size 0.6) (drill 0.3) (layers "F.Cu" "B.Cu") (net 1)))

